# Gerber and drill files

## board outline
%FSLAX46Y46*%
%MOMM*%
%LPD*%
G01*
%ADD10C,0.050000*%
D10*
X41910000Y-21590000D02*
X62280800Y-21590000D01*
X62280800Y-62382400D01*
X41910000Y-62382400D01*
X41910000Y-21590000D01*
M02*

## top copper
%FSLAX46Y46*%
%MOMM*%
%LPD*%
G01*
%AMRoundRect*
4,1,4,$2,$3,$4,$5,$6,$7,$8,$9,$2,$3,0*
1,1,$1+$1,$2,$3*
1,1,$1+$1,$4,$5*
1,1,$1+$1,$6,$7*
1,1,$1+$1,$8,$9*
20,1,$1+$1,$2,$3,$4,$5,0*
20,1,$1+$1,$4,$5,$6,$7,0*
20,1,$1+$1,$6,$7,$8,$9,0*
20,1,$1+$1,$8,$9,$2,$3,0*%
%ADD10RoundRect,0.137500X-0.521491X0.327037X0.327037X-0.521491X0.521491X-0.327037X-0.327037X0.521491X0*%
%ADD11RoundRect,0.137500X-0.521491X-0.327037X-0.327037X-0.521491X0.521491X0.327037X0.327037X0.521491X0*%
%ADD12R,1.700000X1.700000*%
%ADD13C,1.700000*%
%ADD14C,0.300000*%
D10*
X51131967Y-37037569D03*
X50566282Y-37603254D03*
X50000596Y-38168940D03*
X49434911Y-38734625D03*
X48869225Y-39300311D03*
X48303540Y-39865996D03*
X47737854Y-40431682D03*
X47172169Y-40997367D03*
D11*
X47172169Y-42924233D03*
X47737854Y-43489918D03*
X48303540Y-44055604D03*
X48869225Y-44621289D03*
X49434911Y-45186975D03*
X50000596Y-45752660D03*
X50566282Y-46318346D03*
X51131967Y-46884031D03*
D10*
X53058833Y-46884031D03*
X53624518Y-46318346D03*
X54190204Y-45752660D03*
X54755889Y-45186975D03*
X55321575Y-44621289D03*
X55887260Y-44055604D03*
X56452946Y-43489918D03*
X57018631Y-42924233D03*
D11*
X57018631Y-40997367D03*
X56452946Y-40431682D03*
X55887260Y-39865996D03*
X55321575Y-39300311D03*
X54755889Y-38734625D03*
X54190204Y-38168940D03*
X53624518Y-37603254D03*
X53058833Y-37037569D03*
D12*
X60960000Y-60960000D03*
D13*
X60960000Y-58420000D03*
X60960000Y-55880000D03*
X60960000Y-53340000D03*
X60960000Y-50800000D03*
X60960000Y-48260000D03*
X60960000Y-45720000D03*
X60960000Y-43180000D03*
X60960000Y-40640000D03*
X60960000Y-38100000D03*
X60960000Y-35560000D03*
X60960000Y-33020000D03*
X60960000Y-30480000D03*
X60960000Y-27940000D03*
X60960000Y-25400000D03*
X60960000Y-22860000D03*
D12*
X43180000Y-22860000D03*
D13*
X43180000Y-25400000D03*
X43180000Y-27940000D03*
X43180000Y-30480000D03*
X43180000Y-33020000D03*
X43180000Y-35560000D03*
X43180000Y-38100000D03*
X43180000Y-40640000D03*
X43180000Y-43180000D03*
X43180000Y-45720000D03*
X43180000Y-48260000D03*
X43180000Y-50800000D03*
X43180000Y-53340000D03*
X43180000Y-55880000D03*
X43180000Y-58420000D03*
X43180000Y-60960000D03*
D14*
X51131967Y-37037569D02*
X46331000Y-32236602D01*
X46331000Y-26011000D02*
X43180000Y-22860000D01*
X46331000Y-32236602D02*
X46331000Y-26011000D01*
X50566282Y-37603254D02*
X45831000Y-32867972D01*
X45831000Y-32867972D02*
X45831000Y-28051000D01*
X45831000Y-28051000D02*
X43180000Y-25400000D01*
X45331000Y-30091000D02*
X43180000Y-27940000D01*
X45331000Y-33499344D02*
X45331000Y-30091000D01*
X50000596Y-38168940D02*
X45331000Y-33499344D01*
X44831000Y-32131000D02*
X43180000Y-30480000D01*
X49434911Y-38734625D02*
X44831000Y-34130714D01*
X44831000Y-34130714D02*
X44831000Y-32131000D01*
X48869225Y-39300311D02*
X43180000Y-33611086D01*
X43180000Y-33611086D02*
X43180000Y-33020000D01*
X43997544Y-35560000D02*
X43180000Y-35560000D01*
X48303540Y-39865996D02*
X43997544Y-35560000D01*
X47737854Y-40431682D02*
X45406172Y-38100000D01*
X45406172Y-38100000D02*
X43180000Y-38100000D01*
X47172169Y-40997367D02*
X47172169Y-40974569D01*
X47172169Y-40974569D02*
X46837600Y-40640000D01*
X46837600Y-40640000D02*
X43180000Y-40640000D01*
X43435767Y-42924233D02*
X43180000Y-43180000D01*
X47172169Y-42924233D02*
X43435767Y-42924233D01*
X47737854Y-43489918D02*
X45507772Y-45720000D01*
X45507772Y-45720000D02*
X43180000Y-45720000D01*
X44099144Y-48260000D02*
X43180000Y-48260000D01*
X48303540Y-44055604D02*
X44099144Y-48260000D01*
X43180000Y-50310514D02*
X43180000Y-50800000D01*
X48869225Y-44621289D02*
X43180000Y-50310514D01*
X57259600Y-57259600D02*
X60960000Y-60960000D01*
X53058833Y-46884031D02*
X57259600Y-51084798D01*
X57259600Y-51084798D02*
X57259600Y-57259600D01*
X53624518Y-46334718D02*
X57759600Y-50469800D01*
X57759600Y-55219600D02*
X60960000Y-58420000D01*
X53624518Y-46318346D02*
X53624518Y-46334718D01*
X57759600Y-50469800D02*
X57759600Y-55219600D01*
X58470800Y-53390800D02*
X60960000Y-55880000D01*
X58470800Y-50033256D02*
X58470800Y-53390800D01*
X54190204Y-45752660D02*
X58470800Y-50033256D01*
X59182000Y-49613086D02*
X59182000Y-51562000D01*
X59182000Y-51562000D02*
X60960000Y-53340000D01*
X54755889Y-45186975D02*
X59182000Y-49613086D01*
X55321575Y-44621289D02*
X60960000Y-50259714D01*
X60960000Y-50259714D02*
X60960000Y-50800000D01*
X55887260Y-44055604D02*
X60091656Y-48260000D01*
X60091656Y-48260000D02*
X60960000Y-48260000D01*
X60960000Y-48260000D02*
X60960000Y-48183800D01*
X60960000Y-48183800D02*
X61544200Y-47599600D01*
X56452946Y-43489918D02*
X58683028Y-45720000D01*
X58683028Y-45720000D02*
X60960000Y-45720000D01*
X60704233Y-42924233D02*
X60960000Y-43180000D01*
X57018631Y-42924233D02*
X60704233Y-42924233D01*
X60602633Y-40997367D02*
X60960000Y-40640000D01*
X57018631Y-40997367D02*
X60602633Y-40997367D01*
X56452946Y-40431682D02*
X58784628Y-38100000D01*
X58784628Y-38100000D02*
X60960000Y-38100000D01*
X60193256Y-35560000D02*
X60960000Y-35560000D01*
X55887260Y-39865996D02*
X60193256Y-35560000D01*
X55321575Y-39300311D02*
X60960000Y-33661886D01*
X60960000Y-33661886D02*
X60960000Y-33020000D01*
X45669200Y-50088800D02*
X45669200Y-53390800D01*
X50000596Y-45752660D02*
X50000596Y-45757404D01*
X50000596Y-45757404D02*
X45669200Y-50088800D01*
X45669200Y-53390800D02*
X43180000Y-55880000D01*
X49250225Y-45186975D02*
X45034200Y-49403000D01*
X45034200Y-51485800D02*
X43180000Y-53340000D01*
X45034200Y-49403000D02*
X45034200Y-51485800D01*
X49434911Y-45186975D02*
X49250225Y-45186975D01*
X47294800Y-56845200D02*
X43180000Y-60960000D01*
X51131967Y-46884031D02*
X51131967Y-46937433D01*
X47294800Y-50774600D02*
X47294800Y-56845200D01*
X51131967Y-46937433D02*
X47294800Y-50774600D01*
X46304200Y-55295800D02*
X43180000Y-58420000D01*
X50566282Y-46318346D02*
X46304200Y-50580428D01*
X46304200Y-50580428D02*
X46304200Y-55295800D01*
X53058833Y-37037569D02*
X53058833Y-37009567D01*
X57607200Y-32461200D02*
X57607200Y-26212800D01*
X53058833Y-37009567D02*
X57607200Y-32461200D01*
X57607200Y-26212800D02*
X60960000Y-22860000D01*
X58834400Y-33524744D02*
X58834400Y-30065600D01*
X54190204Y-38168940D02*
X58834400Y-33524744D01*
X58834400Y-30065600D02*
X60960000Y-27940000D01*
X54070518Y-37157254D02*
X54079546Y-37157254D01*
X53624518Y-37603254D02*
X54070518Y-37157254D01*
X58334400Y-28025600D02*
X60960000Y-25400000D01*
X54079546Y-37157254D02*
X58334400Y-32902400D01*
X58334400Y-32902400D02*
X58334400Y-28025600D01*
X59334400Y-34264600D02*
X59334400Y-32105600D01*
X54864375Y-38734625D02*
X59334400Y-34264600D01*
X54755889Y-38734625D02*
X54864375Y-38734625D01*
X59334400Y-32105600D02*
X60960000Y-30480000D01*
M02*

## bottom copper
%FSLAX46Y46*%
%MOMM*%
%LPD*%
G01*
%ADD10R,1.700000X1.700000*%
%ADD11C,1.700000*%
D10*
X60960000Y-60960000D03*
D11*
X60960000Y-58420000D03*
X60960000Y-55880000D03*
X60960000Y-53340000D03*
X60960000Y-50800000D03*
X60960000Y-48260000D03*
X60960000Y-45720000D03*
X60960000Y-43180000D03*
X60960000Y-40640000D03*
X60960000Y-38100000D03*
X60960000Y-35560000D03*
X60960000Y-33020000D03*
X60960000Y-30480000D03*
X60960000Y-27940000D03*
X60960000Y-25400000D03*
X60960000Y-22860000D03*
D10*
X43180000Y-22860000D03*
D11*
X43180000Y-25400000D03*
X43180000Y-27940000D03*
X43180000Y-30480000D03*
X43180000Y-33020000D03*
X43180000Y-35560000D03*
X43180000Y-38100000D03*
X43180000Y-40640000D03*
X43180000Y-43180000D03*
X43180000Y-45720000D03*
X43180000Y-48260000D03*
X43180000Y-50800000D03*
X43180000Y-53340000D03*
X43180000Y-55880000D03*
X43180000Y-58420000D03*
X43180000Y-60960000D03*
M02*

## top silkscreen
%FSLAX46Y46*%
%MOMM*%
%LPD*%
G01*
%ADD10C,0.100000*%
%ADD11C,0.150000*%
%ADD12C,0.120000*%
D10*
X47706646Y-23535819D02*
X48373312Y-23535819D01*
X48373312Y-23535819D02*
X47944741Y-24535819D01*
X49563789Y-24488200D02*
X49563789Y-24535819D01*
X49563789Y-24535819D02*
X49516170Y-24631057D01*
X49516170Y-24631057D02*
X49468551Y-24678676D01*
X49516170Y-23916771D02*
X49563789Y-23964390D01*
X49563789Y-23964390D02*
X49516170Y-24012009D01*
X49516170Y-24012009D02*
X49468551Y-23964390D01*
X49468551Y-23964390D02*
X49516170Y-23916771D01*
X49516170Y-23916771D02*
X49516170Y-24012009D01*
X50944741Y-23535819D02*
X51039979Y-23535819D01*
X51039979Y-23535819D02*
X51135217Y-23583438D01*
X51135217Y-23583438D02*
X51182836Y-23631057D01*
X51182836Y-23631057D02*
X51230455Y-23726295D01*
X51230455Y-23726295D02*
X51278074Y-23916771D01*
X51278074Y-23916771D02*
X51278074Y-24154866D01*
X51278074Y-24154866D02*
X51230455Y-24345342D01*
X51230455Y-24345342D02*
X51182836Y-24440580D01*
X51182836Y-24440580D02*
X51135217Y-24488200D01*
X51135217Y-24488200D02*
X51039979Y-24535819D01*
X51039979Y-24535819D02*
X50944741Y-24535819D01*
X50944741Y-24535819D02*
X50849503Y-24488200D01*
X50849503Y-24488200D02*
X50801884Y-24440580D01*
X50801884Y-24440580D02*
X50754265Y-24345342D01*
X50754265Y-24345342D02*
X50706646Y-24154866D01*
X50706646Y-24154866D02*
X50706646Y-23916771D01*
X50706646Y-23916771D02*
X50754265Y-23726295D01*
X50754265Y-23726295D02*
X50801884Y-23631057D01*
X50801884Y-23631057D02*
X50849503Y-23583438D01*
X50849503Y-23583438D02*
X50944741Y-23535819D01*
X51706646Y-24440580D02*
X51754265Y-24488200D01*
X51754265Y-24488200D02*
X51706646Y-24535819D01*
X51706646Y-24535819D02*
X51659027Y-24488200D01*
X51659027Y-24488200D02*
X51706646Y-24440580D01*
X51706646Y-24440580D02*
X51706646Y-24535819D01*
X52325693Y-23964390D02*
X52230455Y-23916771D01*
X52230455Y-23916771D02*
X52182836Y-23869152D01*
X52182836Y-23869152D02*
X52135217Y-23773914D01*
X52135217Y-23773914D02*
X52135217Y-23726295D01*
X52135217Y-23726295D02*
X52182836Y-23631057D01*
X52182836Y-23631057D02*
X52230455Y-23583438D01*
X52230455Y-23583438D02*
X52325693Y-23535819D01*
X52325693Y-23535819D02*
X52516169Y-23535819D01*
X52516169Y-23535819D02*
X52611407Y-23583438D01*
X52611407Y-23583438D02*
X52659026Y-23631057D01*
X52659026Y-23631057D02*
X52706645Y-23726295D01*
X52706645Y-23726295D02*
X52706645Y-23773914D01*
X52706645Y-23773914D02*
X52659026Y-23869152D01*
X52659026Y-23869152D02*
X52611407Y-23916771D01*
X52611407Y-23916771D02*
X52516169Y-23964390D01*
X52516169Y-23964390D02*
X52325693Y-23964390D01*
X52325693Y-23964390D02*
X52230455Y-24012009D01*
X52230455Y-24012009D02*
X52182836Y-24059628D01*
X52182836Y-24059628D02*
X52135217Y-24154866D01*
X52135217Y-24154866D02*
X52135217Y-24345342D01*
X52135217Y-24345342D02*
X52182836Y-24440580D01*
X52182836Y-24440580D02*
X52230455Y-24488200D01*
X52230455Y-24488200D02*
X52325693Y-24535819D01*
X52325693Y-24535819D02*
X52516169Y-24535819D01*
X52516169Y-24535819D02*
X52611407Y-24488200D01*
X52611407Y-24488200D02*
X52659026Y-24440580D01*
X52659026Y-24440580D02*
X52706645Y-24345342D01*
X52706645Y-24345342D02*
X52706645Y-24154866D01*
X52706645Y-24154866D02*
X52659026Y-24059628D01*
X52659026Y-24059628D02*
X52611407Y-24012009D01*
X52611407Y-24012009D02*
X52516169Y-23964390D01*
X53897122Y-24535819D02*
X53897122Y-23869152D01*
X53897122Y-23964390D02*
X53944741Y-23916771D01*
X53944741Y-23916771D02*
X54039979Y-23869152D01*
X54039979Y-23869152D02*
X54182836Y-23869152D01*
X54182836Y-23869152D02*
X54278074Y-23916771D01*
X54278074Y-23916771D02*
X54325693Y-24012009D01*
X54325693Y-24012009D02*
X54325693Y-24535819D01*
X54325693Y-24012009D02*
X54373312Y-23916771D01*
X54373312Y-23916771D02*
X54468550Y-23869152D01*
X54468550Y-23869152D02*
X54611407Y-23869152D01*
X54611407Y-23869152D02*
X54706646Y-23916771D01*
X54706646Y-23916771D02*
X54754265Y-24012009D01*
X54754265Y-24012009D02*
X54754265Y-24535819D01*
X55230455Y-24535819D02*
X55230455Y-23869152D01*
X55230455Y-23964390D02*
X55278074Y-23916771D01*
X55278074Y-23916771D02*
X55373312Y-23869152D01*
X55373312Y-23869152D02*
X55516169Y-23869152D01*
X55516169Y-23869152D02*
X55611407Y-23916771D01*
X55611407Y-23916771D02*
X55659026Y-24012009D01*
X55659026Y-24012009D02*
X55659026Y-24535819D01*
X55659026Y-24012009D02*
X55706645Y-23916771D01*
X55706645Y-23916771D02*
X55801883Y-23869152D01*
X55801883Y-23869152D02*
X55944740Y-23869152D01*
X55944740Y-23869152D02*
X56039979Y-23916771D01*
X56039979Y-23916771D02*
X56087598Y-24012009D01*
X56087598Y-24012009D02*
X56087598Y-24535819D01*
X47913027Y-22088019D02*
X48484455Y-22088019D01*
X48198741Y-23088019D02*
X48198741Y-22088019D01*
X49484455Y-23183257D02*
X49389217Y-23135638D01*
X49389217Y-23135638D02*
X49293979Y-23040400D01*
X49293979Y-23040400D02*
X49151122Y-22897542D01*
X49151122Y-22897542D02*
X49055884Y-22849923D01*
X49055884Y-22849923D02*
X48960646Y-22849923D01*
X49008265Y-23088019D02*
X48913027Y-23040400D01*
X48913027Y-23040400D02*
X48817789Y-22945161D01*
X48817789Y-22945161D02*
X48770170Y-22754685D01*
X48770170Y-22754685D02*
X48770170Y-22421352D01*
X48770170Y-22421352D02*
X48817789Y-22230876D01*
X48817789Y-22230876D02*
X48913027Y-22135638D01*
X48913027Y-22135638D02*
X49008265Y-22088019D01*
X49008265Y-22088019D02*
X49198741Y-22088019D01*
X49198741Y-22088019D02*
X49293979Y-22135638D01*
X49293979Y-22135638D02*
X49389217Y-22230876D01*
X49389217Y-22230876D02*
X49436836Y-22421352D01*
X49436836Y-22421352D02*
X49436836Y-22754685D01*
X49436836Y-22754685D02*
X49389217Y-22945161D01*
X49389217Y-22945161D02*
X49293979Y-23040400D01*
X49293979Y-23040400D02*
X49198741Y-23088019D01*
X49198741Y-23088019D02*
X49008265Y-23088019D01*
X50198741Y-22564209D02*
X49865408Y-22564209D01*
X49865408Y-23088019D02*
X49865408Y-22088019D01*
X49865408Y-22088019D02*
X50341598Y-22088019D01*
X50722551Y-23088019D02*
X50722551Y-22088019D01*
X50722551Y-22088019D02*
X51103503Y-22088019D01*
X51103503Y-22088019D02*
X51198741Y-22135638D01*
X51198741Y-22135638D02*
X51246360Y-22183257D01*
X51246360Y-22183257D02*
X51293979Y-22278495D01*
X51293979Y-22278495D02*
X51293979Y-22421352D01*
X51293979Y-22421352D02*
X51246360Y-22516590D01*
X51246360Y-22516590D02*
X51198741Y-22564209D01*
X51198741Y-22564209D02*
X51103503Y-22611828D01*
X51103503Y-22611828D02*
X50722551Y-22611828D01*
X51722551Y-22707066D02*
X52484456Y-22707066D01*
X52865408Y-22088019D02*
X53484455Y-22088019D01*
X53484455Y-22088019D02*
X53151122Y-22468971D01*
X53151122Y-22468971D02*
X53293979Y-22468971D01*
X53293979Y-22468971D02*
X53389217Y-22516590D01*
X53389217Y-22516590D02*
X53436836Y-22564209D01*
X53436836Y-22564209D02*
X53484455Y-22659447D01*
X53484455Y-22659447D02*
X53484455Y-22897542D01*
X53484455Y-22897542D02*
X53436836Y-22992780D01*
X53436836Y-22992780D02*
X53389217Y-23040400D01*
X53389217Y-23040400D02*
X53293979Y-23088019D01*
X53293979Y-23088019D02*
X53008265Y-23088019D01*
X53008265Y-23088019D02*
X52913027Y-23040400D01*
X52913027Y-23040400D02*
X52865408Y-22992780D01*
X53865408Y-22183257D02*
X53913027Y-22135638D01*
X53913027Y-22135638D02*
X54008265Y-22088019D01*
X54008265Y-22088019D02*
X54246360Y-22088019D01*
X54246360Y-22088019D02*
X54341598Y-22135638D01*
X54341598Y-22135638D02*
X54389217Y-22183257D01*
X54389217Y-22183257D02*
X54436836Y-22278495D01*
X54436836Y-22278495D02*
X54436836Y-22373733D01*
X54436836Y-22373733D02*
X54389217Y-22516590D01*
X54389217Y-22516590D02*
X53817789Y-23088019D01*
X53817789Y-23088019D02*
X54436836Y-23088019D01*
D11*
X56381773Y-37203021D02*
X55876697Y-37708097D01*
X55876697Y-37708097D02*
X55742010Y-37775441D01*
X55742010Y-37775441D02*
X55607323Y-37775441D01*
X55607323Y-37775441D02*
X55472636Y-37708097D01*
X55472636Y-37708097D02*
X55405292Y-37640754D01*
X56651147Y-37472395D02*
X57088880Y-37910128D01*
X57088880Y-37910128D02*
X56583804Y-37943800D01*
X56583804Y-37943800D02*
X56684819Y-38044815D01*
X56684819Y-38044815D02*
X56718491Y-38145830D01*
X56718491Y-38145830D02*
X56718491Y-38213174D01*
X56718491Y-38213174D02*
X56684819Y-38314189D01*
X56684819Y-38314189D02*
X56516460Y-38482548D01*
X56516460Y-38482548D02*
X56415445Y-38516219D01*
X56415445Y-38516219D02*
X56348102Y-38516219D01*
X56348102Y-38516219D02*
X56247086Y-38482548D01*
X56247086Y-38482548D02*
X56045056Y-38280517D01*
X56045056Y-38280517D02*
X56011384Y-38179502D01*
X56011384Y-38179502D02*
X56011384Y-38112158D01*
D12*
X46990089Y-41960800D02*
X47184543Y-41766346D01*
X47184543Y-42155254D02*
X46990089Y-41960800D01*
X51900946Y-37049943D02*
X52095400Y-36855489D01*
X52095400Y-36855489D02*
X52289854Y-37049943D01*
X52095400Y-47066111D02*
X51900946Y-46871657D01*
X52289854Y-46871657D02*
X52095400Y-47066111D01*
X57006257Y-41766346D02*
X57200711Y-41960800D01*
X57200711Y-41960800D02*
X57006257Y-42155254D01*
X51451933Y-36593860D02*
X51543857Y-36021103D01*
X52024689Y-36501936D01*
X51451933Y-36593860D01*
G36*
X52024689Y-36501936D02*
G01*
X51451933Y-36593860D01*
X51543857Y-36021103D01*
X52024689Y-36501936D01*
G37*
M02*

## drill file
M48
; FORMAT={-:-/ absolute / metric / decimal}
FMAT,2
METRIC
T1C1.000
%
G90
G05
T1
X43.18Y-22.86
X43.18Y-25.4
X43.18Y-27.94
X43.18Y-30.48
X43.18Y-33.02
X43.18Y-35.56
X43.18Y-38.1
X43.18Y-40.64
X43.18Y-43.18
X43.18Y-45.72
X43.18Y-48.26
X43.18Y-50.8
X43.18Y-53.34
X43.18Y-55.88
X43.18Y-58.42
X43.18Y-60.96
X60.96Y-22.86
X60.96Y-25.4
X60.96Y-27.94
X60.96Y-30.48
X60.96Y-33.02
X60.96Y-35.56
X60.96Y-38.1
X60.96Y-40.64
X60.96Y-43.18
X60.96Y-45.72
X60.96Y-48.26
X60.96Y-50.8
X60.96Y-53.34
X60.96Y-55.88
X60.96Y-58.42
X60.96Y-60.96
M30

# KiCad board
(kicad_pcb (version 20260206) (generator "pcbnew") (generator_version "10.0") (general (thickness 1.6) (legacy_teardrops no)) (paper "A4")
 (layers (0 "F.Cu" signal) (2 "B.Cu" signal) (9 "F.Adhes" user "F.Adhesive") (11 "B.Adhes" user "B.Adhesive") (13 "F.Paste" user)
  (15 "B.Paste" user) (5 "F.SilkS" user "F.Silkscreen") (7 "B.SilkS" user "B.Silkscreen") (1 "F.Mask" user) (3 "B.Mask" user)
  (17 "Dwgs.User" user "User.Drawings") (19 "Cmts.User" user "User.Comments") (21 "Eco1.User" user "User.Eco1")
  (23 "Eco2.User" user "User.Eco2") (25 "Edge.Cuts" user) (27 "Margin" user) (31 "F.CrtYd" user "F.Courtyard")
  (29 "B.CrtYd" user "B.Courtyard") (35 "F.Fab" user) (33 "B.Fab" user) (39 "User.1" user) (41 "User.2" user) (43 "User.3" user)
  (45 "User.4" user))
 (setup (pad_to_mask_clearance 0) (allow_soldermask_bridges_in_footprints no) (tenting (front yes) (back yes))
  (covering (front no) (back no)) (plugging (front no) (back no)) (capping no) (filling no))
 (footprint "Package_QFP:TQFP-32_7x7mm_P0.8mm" (layer "F.Cu") (at 52.0954 41.9608 -45)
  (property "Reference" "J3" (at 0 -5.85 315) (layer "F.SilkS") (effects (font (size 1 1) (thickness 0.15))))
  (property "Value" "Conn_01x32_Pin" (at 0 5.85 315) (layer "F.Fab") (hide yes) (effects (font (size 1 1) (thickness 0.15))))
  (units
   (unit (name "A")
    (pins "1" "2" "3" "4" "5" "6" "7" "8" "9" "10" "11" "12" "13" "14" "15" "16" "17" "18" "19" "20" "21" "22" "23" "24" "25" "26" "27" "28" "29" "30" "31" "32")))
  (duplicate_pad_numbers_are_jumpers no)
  (fp_line (start -3.61 3.61) (end -3.61 3.335001) (stroke (width 0.12) (type solid)) (layer "F.SilkS"))
  (fp_line (start -3.335001 3.61) (end -3.61 3.61) (stroke (width 0.12) (type solid)) (layer "F.SilkS"))
  (fp_line (start -3.61 -3.335001) (end -3.61 -3.61) (stroke (width 0.12) (type solid)) (layer "F.SilkS"))
  (fp_line (start -3.61 -3.61) (end -3.335001 -3.61) (stroke (width 0.12) (type solid)) (layer "F.SilkS"))
  (fp_line (start 3.61 3.61) (end 3.335001 3.61) (stroke (width 0.12) (type solid)) (layer "F.SilkS"))
  (fp_line (start 3.61 3.335001) (end 3.61 3.61) (stroke (width 0.12) (type solid)) (layer "F.SilkS"))
  (fp_line (start 3.335001 -3.61) (end 3.61 -3.61) (stroke (width 0.12) (type solid)) (layer "F.SilkS"))
  (fp_line (start 3.61 -3.61) (end 3.61 -3.335001) (stroke (width 0.12) (type solid)) (layer "F.SilkS"))
  (fp_poly (pts (xy -4.25 -3.34) (xy -4.59 -3.81) (xy -3.91 -3.81)) (stroke (width 0.12) (type solid)) (fill yes) (layer "F.SilkS"))
  (pad "1" smd roundrect (at -4.1625 -2.8 315) (size 1.475 0.55) (layers "F.Cu" "F.Mask" "F.Paste") (roundrect_rratio 0.25)
   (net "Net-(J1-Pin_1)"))
  (pad "2" smd roundrect (at -4.1625 -2.000001 315) (size 1.475 0.55) (layers "F.Cu" "F.Mask" "F.Paste") (roundrect_rratio 0.25)
   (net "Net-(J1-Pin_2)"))
  (pad "3" smd roundrect (at -4.1625 -1.2 315) (size 1.475 0.55) (layers "F.Cu" "F.Mask" "F.Paste") (roundrect_rratio 0.25)
   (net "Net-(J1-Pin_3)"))
  (pad "4" smd roundrect (at -4.1625 -0.4 315) (size 1.475 0.55) (layers "F.Cu" "F.Mask" "F.Paste") (roundrect_rratio 0.25)
   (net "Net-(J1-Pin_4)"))
  (pad "5" smd roundrect (at -4.1625 0.4 315) (size 1.475 0.55) (layers "F.Cu" "F.Mask" "F.Paste") (roundrect_rratio 0.25)
   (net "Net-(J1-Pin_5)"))
  (pad "6" smd roundrect (at -4.1625 1.2 315) (size 1.475 0.55) (layers "F.Cu" "F.Mask" "F.Paste") (roundrect_rratio 0.25)
   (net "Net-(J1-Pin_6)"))
  (pad "7" smd roundrect (at -4.1625 2.000001 315) (size 1.475 0.55) (layers "F.Cu" "F.Mask" "F.Paste") (roundrect_rratio 0.25)
   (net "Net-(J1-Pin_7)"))
  (pad "8" smd roundrect (at -4.1625 2.8 315) (size 1.475 0.55) (layers "F.Cu" "F.Mask" "F.Paste") (roundrect_rratio 0.25)
   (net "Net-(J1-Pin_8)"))
  (pad "9" smd roundrect (at -2.8 4.1625 315) (size 0.55 1.475) (layers "F.Cu" "F.Mask" "F.Paste") (roundrect_rratio 0.25)
   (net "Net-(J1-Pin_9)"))
  (pad "10" smd roundrect (at -2.000001 4.1625 315) (size 0.55 1.475) (layers "F.Cu" "F.Mask" "F.Paste") (roundrect_rratio 0.25)
   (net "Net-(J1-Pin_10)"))
  (pad "11" smd roundrect (at -1.2 4.1625 315) (size 0.55 1.475) (layers "F.Cu" "F.Mask" "F.Paste") (roundrect_rratio 0.25)
   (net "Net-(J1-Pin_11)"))
  (pad "12" smd roundrect (at -0.4 4.1625 315) (size 0.55 1.475) (layers "F.Cu" "F.Mask" "F.Paste") (roundrect_rratio 0.25)
   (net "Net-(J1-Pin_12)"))
  (pad "13" smd roundrect (at 0.4 4.1625 315) (size 0.55 1.475) (layers "F.Cu" "F.Mask" "F.Paste") (roundrect_rratio 0.25)
   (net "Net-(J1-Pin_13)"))
  (pad "14" smd roundrect (at 1.2 4.1625 315) (size 0.55 1.475) (layers "F.Cu" "F.Mask" "F.Paste") (roundrect_rratio 0.25)
   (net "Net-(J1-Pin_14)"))
  (pad "15" smd roundrect (at 2.000001 4.1625 315) (size 0.55 1.475) (layers "F.Cu" "F.Mask" "F.Paste") (roundrect_rratio 0.25)
   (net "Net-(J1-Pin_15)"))
  (pad "16" smd roundrect (at 2.8 4.1625 315) (size 0.55 1.475) (layers "F.Cu" "F.Mask" "F.Paste") (roundrect_rratio 0.25)
   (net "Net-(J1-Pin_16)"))
  (pad "17" smd roundrect (at 4.1625 2.8 315) (size 1.475 0.55) (layers "F.Cu" "F.Mask" "F.Paste") (roundrect_rratio 0.25)
   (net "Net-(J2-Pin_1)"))
  (pad "18" smd roundrect (at 4.1625 2.000001 315) (size 1.475 0.55) (layers "F.Cu" "F.Mask" "F.Paste") (roundrect_rratio 0.25)
   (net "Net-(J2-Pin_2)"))
  (pad "19" smd roundrect (at 4.1625 1.2 315) (size 1.475 0.55) (layers "F.Cu" "F.Mask" "F.Paste") (roundrect_rratio 0.25)
   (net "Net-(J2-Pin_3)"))
  (pad "20" smd roundrect (at 4.1625 0.4 315) (size 1.475 0.55) (layers "F.Cu" "F.Mask" "F.Paste") (roundrect_rratio 0.25)
   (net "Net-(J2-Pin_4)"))
  (pad "21" smd roundrect (at 4.1625 -0.4 315) (size 1.475 0.55) (layers "F.Cu" "F.Mask" "F.Paste") (roundrect_rratio 0.25)
   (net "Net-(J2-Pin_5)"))
  (pad "22" smd roundrect (at 4.1625 -1.2 315) (size 1.475 0.55) (layers "F.Cu" "F.Mask" "F.Paste") (roundrect_rratio 0.25)
   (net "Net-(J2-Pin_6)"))
  (pad "23" smd roundrect (at 4.1625 -2.000001 315) (size 1.475 0.55) (layers "F.Cu" "F.Mask" "F.Paste") (roundrect_rratio 0.25)
   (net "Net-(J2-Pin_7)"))
  (pad "24" smd roundrect (at 4.1625 -2.8 315) (size 1.475 0.55) (layers "F.Cu" "F.Mask" "F.Paste") (roundrect_rratio 0.25)
   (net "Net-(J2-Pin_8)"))
  (pad "25" smd roundrect (at 2.8 -4.1625 315) (size 0.55 1.475) (layers "F.Cu" "F.Mask" "F.Paste") (roundrect_rratio 0.25)
   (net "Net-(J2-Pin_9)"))
  (pad "26" smd roundrect (at 2.000001 -4.1625 315) (size 0.55 1.475) (layers "F.Cu" "F.Mask" "F.Paste") (roundrect_rratio 0.25)
   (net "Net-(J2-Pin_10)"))
  (pad "27" smd roundrect (at 1.2 -4.1625 315) (size 0.55 1.475) (layers "F.Cu" "F.Mask" "F.Paste") (roundrect_rratio 0.25)
   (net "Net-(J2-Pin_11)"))
  (pad "28" smd roundrect (at 0.4 -4.1625 315) (size 0.55 1.475) (layers "F.Cu" "F.Mask" "F.Paste") (roundrect_rratio 0.25)
   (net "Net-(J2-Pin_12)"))
  (pad "29" smd roundrect (at -0.4 -4.1625 315) (size 0.55 1.475) (layers "F.Cu" "F.Mask" "F.Paste") (roundrect_rratio 0.25)
   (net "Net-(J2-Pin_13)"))
  (pad "30" smd roundrect (at -1.2 -4.1625 315) (size 0.55 1.475) (layers "F.Cu" "F.Mask" "F.Paste") (roundrect_rratio 0.25)
   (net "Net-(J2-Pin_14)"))
  (pad "31" smd roundrect (at -2.000001 -4.1625 315) (size 0.55 1.475) (layers "F.Cu" "F.Mask" "F.Paste") (roundrect_rratio 0.25)
   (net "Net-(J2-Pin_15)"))
  (pad "32" smd roundrect (at -2.8 -4.1625 315) (size 0.55 1.475) (layers "F.Cu" "F.Mask" "F.Paste") (roundrect_rratio 0.25)
   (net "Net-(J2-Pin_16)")))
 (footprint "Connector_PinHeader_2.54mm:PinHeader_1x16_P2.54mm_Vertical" (layer "B.Cu") (at 60.96 60.96)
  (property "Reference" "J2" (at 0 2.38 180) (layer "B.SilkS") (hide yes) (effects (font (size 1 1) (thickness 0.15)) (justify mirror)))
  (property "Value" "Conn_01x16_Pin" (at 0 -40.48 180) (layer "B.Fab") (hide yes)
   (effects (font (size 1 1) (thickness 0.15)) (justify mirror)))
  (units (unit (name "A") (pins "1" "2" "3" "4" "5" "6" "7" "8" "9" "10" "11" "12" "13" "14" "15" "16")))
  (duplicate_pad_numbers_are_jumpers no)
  (pad "1" thru_hole rect (at 0 0) (size 1.7 1.7) (drill 1) (layers "*.Cu" "*.Mask") (remove_unused_layers no) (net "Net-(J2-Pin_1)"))
  (pad "2" thru_hole circle (at 0 -2.54) (size 1.7 1.7) (drill 1) (layers "*.Cu" "*.Mask") (remove_unused_layers no) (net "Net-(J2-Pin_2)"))
  (pad "3" thru_hole circle (at 0 -5.08) (size 1.7 1.7) (drill 1) (layers "*.Cu" "*.Mask") (remove_unused_layers no) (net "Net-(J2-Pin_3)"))
  (pad "4" thru_hole circle (at 0 -7.62) (size 1.7 1.7) (drill 1) (layers "*.Cu" "*.Mask") (remove_unused_layers no) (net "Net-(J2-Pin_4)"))
  (pad "5" thru_hole circle (at 0 -10.16) (size 1.7 1.7) (drill 1) (layers "*.Cu" "*.Mask") (remove_unused_layers no) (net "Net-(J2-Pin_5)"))
  (pad "6" thru_hole circle (at 0 -12.7) (size 1.7 1.7) (drill 1) (layers "*.Cu" "*.Mask") (remove_unused_layers no) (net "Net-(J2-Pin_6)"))
  (pad "7" thru_hole circle (at 0 -15.24) (size 1.7 1.7) (drill 1) (layers "*.Cu" "*.Mask") (remove_unused_layers no) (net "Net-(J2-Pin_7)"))
  (pad "8" thru_hole circle (at 0 -17.78) (size 1.7 1.7) (drill 1) (layers "*.Cu" "*.Mask") (remove_unused_layers no) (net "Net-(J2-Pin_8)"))
  (pad "9" thru_hole circle (at 0 -20.32) (size 1.7 1.7) (drill 1) (layers "*.Cu" "*.Mask") (remove_unused_layers no) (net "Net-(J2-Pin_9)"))
  (pad "10" thru_hole circle (at 0 -22.86) (size 1.7 1.7) (drill 1) (layers "*.Cu" "*.Mask") (remove_unused_layers no)
   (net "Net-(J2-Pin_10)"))
  (pad "11" thru_hole circle (at 0 -25.4) (size 1.7 1.7) (drill 1) (layers "*.Cu" "*.Mask") (remove_unused_layers no)
   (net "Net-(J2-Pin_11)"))
  (pad "12" thru_hole circle (at 0 -27.94) (size 1.7 1.7) (drill 1) (layers "*.Cu" "*.Mask") (remove_unused_layers no)
   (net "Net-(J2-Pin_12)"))
  (pad "13" thru_hole circle (at 0 -30.48) (size 1.7 1.7) (drill 1) (layers "*.Cu" "*.Mask") (remove_unused_layers no)
   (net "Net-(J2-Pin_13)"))
  (pad "14" thru_hole circle (at 0 -33.02) (size 1.7 1.7) (drill 1) (layers "*.Cu" "*.Mask") (remove_unused_layers no)
   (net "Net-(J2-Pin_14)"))
  (pad "15" thru_hole circle (at 0 -35.56) (size 1.7 1.7) (drill 1) (layers "*.Cu" "*.Mask") (remove_unused_layers no)
   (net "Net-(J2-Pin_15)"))
  (pad "16" thru_hole circle (at 0 -38.1) (size 1.7 1.7) (drill 1) (layers "*.Cu" "*.Mask") (remove_unused_layers no)
   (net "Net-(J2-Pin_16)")))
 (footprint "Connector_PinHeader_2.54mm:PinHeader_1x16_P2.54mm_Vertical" (layer "B.Cu") (at 43.18 22.86 180)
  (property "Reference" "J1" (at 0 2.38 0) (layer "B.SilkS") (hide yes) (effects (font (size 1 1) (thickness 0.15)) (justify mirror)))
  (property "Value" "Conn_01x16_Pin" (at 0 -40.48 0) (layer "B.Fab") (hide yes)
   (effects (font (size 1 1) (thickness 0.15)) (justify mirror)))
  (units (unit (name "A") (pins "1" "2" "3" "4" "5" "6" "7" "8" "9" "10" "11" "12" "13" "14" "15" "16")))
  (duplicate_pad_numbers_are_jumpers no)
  (pad "1" thru_hole rect (at 0 0 180) (size 1.7 1.7) (drill 1) (layers "*.Cu" "*.Mask") (remove_unused_layers no) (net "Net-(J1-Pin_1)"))
  (pad "2" thru_hole circle (at 0 -2.54 180) (size 1.7 1.7) (drill 1) (layers "*.Cu" "*.Mask") (remove_unused_layers no)
   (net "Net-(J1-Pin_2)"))
  (pad "3" thru_hole circle (at 0 -5.08 180) (size 1.7 1.7) (drill 1) (layers "*.Cu" "*.Mask") (remove_unused_layers no)
   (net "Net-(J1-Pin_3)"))
  (pad "4" thru_hole circle (at 0 -7.62 180) (size 1.7 1.7) (drill 1) (layers "*.Cu" "*.Mask") (remove_unused_layers no)
   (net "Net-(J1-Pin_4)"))
  (pad "5" thru_hole circle (at 0 -10.16 180) (size 1.7 1.7) (drill 1) (layers "*.Cu" "*.Mask") (remove_unused_layers no)
   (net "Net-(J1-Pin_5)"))
  (pad "6" thru_hole circle (at 0 -12.7 180) (size 1.7 1.7) (drill 1) (layers "*.Cu" "*.Mask") (remove_unused_layers no)
   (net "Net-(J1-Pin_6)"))
  (pad "7" thru_hole circle (at 0 -15.24 180) (size 1.7 1.7) (drill 1) (layers "*.Cu" "*.Mask") (remove_unused_layers no)
   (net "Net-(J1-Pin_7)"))
  (pad "8" thru_hole circle (at 0 -17.78 180) (size 1.7 1.7) (drill 1) (layers "*.Cu" "*.Mask") (remove_unused_layers no)
   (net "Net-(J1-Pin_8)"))
  (pad "9" thru_hole circle (at 0 -20.32 180) (size 1.7 1.7) (drill 1) (layers "*.Cu" "*.Mask") (remove_unused_layers no)
   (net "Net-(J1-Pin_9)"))
  (pad "10" thru_hole circle (at 0 -22.86 180) (size 1.7 1.7) (drill 1) (layers "*.Cu" "*.Mask") (remove_unused_layers no)
   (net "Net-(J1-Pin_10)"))
  (pad "11" thru_hole circle (at 0 -25.4 180) (size 1.7 1.7) (drill 1) (layers "*.Cu" "*.Mask") (remove_unused_layers no)
   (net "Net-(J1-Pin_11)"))
  (pad "12" thru_hole circle (at 0 -27.94 180) (size 1.7 1.7) (drill 1) (layers "*.Cu" "*.Mask") (remove_unused_layers no)
   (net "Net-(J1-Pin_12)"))
  (pad "13" thru_hole circle (at 0 -30.48 180) (size 1.7 1.7) (drill 1) (layers "*.Cu" "*.Mask") (remove_unused_layers no)
   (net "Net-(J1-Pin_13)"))
  (pad "14" thru_hole circle (at 0 -33.02 180) (size 1.7 1.7) (drill 1) (layers "*.Cu" "*.Mask") (remove_unused_layers no)
   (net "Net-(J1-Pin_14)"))
  (pad "15" thru_hole circle (at 0 -35.56 180) (size 1.7 1.7) (drill 1) (layers "*.Cu" "*.Mask") (remove_unused_layers no)
   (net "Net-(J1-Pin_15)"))
  (pad "16" thru_hole circle (at 0 -38.1 180) (size 1.7 1.7) (drill 1) (layers "*.Cu" "*.Mask") (remove_unused_layers no)
   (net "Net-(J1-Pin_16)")))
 (gr_rect (start 41.91 21.59) (end 62.2808 62.3824) (stroke (width 0.05) (type default)) (fill no) (layer "Edge.Cuts"))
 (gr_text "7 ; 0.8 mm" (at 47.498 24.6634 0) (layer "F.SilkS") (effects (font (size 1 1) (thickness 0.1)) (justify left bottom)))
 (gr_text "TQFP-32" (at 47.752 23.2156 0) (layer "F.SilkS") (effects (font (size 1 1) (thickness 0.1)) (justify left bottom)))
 (segment (start 51.131967 37.037569) (end 46.331 32.236602) (width 0.3) (layer "F.Cu") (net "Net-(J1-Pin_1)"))
 (segment (start 46.331 26.011) (end 43.18 22.86) (width 0.3) (layer "F.Cu") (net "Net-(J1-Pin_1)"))
 (segment (start 46.331 32.236602) (end 46.331 26.011) (width 0.3) (layer "F.Cu") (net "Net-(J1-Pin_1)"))
 (segment (start 50.566282 37.603254) (end 45.831 32.867972) (width 0.3) (layer "F.Cu") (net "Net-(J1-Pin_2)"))
 (segment (start 45.831 32.867972) (end 45.831 28.051) (width 0.3) (layer "F.Cu") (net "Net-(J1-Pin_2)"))
 (segment (start 45.831 28.051) (end 43.18 25.4) (width 0.3) (layer "F.Cu") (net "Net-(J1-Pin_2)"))
 (segment (start 45.331 30.091) (end 43.18 27.94) (width 0.3) (layer "F.Cu") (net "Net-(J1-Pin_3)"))
 (segment (start 45.331 33.499344) (end 45.331 30.091) (width 0.3) (layer "F.Cu") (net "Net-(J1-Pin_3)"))
 (segment (start 50.000596 38.16894) (end 45.331 33.499344) (width 0.3) (layer "F.Cu") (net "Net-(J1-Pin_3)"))
 (segment (start 44.831 32.131) (end 43.18 30.48) (width 0.3) (layer "F.Cu") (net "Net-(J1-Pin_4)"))
 (segment (start 49.434911 38.734625) (end 44.831 34.130714) (width 0.3) (layer "F.Cu") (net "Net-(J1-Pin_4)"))
 (segment (start 44.831 34.130714) (end 44.831 32.131) (width 0.3) (layer "F.Cu") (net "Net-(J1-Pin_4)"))
 (segment (start 48.869225 39.300311) (end 43.18 33.611086) (width 0.3) (layer "F.Cu") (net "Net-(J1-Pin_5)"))
 (segment (start 43.18 33.611086) (end 43.18 33.02) (width 0.3) (layer "F.Cu") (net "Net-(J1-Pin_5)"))
 (segment (start 43.997544 35.56) (end 43.18 35.56) (width 0.3) (layer "F.Cu") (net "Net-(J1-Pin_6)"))
 (segment (start 48.30354 39.865996) (end 43.997544 35.56) (width 0.3) (layer "F.Cu") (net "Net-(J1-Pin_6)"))
 (segment (start 47.737854 40.431682) (end 45.406172 38.1) (width 0.3) (layer "F.Cu") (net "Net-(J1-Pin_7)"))
 (segment (start 45.406172 38.1) (end 43.18 38.1) (width 0.3) (layer "F.Cu") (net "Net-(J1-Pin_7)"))
 (segment (start 47.172169 40.997367) (end 47.172169 40.974569) (width 0.3) (layer "F.Cu") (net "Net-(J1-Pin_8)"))
 (segment (start 47.172169 40.974569) (end 46.8376 40.64) (width 0.3) (layer "F.Cu") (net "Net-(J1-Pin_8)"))
 (segment (start 46.8376 40.64) (end 43.18 40.64) (width 0.3) (layer "F.Cu") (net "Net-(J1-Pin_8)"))
 (segment (start 43.435767 42.924233) (end 43.18 43.18) (width 0.3) (layer "F.Cu") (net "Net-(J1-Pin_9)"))
 (segment (start 47.172169 42.924233) (end 43.435767 42.924233) (width 0.3) (layer "F.Cu") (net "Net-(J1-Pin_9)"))
 (segment (start 47.737854 43.489918) (end 45.507772 45.72) (width 0.3) (layer "F.Cu") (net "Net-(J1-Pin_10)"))
 (segment (start 45.507772 45.72) (end 43.18 45.72) (width 0.3) (layer "F.Cu") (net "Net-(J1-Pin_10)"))
 (segment (start 44.099144 48.26) (end 43.18 48.26) (width 0.3) (layer "F.Cu") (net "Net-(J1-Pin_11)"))
 (segment (start 48.30354 44.055604) (end 44.099144 48.26) (width 0.3) (layer "F.Cu") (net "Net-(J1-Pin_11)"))
 (segment (start 43.18 50.310514) (end 43.18 50.8) (width 0.3) (layer "F.Cu") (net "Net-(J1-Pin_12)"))
 (segment (start 48.869225 44.621289) (end 43.18 50.310514) (width 0.3) (layer "F.Cu") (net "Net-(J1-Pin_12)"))
 (segment (start 57.2596 57.2596) (end 60.96 60.96) (width 0.3) (layer "F.Cu") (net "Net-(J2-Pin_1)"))
 (segment (start 53.058833 46.884031) (end 57.2596 51.084798) (width 0.3) (layer "F.Cu") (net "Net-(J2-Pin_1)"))
 (segment (start 57.2596 51.084798) (end 57.2596 57.2596) (width 0.3) (layer "F.Cu") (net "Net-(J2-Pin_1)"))
 (segment (start 53.624518 46.334718) (end 57.7596 50.4698) (width 0.3) (layer "F.Cu") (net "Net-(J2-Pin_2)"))
 (segment (start 57.7596 55.2196) (end 60.96 58.42) (width 0.3) (layer "F.Cu") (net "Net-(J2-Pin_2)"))
 (segment (start 53.624518 46.318346) (end 53.624518 46.334718) (width 0.3) (layer "F.Cu") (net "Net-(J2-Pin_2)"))
 (segment (start 57.7596 50.4698) (end 57.7596 55.2196) (width 0.3) (layer "F.Cu") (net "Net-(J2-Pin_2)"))
 (segment (start 58.4708 53.3908) (end 60.96 55.88) (width 0.3) (layer "F.Cu") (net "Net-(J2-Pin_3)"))
 (segment (start 58.4708 50.033256) (end 58.4708 53.3908) (width 0.3) (layer "F.Cu") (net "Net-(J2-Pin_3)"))
 (segment (start 54.190204 45.75266) (end 58.4708 50.033256) (width 0.3) (layer "F.Cu") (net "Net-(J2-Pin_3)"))
 (segment (start 59.182 49.613086) (end 59.182 51.562) (width 0.3) (layer "F.Cu") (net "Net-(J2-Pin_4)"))
 (segment (start 59.182 51.562) (end 60.96 53.34) (width 0.3) (layer "F.Cu") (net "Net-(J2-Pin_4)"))
 (segment (start 54.755889 45.186975) (end 59.182 49.613086) (width 0.3) (layer "F.Cu") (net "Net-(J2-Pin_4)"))
 (segment (start 55.321575 44.621289) (end 60.96 50.259714) (width 0.3) (layer "F.Cu") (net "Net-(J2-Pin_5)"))
 (segment (start 60.96 50.259714) (end 60.96 50.8) (width 0.3) (layer "F.Cu") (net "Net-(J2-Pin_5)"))
 (segment (start 55.88726 44.055604) (end 60.091656 48.26) (width 0.3) (layer "F.Cu") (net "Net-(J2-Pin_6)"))
 (segment (start 60.091656 48.26) (end 60.96 48.26) (width 0.3) (layer "F.Cu") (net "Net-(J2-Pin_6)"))
 (segment (start 60.96 48.26) (end 60.96 48.1838) (width 0.3) (layer "F.Cu") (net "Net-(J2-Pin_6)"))
 (segment (start 60.96 48.1838) (end 61.5442 47.5996) (width 0.3) (layer "F.Cu") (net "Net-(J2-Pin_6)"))
 (segment (start 56.452946 43.489918) (end 58.683028 45.72) (width 0.3) (layer "F.Cu") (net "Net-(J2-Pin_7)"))
 (segment (start 58.683028 45.72) (end 60.96 45.72) (width 0.3) (layer "F.Cu") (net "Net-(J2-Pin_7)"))
 (segment (start 60.704233 42.924233) (end 60.96 43.18) (width 0.3) (layer "F.Cu") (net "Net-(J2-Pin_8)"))
 (segment (start 57.018631 42.924233) (end 60.704233 42.924233) (width 0.3) (layer "F.Cu") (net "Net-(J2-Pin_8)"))
 (segment (start 60.602633 40.997367) (end 60.96 40.64) (width 0.3) (layer "F.Cu") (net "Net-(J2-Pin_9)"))
 (segment (start 57.018631 40.997367) (end 60.602633 40.997367) (width 0.3) (layer "F.Cu") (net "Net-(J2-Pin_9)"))
 (segment (start 56.452946 40.431682) (end 58.784628 38.1) (width 0.3) (layer "F.Cu") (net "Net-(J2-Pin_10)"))
 (segment (start 58.784628 38.1) (end 60.96 38.1) (width 0.3) (layer "F.Cu") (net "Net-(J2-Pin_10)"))
 (segment (start 60.193256 35.56) (end 60.96 35.56) (width 0.3) (layer "F.Cu") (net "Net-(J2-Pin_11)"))
 (segment (start 55.88726 39.865996) (end 60.193256 35.56) (width 0.3) (layer "F.Cu") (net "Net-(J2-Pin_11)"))
 (segment (start 55.321575 39.300311) (end 60.96 33.661886) (width 0.3) (layer "F.Cu") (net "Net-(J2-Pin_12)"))
 (segment (start 60.96 33.661886) (end 60.96 33.02) (width 0.3) (layer "F.Cu") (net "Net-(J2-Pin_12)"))
 (segment (start 45.6692 50.0888) (end 45.6692 53.3908) (width 0.3) (layer "F.Cu") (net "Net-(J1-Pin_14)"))
 (segment (start 50.000596 45.75266) (end 50.000596 45.757404) (width 0.3) (layer "F.Cu") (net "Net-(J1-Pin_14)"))
 (segment (start 50.000596 45.757404) (end 45.6692 50.0888) (width 0.3) (layer "F.Cu") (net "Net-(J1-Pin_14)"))
 (segment (start 45.6692 53.3908) (end 43.18 55.88) (width 0.3) (layer "F.Cu") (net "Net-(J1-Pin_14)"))
 (segment (start 49.250225 45.186975) (end 45.0342 49.403) (width 0.3) (layer "F.Cu") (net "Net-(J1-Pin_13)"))
 (segment (start 45.0342 51.4858) (end 43.18 53.34) (width 0.3) (layer "F.Cu") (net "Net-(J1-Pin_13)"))
 (segment (start 45.0342 49.403) (end 45.0342 51.4858) (width 0.3) (layer "F.Cu") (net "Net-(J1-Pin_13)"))
 (segment (start 49.434911 45.186975) (end 49.250225 45.186975) (width 0.3) (layer "F.Cu") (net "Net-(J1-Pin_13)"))
 (segment (start 47.2948 56.8452) (end 43.18 60.96) (width 0.3) (layer "F.Cu") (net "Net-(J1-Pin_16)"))
 (segment (start 51.131967 46.884031) (end 51.131967 46.937433) (width 0.3) (layer "F.Cu") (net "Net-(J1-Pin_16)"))
 (segment (start 47.2948 50.7746) (end 47.2948 56.8452) (width 0.3) (layer "F.Cu") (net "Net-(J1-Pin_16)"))
 (segment (start 51.131967 46.937433) (end 47.2948 50.7746) (width 0.3) (layer "F.Cu") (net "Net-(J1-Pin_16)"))
 (segment (start 46.3042 55.2958) (end 43.18 58.42) (width 0.3) (layer "F.Cu") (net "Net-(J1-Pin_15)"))
 (segment (start 50.566282 46.318346) (end 46.3042 50.580428) (width 0.3) (layer "F.Cu") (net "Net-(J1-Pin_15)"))
 (segment (start 46.3042 50.580428) (end 46.3042 55.2958) (width 0.3) (layer "F.Cu") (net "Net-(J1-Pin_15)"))
 (segment (start 53.058833 37.037569) (end 53.058833 37.009567) (width 0.3) (layer "F.Cu") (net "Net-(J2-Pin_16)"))
 (segment (start 57.6072 32.4612) (end 57.6072 26.2128) (width 0.3) (layer "F.Cu") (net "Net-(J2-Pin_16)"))
 (segment (start 53.058833 37.009567) (end 57.6072 32.4612) (width 0.3) (layer "F.Cu") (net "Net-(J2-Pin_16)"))
 (segment (start 57.6072 26.2128) (end 60.96 22.86) (width 0.3) (layer "F.Cu") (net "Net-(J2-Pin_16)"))
 (segment (start 58.8344 33.524744) (end 58.8344 30.0656) (width 0.3) (layer "F.Cu") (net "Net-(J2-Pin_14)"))
 (segment (start 54.190204 38.16894) (end 58.8344 33.524744) (width 0.3) (layer "F.Cu") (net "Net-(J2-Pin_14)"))
 (segment (start 58.8344 30.0656) (end 60.96 27.94) (width 0.3) (layer "F.Cu") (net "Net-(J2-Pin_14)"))
 (segment (start 54.070518 37.157254) (end 54.079546 37.157254) (width 0.3) (layer "F.Cu") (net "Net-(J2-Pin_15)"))
 (segment (start 53.624518 37.603254) (end 54.070518 37.157254) (width 0.3) (layer "F.Cu") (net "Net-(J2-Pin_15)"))
 (segment (start 58.3344 28.0256) (end 60.96 25.4) (width 0.3) (layer "F.Cu") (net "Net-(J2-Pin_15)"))
 (segment (start 54.079546 37.157254) (end 58.3344 32.9024) (width 0.3) (layer "F.Cu") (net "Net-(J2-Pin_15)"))
 (segment (start 58.3344 32.9024) (end 58.3344 28.0256) (width 0.3) (layer "F.Cu") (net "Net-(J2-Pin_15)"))
 (segment (start 59.3344 34.2646) (end 59.3344 32.1056) (width 0.3) (layer "F.Cu") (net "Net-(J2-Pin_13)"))
 (segment (start 54.864375 38.734625) (end 59.3344 34.2646) (width 0.3) (layer "F.Cu") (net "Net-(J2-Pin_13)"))
 (segment (start 54.755889 38.734625) (end 54.864375 38.734625) (width 0.3) (layer "F.Cu") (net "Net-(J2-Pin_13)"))
 (segment (start 59.3344 32.1056) (end 60.96 30.48) (width 0.3) (layer "F.Cu") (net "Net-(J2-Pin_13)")))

